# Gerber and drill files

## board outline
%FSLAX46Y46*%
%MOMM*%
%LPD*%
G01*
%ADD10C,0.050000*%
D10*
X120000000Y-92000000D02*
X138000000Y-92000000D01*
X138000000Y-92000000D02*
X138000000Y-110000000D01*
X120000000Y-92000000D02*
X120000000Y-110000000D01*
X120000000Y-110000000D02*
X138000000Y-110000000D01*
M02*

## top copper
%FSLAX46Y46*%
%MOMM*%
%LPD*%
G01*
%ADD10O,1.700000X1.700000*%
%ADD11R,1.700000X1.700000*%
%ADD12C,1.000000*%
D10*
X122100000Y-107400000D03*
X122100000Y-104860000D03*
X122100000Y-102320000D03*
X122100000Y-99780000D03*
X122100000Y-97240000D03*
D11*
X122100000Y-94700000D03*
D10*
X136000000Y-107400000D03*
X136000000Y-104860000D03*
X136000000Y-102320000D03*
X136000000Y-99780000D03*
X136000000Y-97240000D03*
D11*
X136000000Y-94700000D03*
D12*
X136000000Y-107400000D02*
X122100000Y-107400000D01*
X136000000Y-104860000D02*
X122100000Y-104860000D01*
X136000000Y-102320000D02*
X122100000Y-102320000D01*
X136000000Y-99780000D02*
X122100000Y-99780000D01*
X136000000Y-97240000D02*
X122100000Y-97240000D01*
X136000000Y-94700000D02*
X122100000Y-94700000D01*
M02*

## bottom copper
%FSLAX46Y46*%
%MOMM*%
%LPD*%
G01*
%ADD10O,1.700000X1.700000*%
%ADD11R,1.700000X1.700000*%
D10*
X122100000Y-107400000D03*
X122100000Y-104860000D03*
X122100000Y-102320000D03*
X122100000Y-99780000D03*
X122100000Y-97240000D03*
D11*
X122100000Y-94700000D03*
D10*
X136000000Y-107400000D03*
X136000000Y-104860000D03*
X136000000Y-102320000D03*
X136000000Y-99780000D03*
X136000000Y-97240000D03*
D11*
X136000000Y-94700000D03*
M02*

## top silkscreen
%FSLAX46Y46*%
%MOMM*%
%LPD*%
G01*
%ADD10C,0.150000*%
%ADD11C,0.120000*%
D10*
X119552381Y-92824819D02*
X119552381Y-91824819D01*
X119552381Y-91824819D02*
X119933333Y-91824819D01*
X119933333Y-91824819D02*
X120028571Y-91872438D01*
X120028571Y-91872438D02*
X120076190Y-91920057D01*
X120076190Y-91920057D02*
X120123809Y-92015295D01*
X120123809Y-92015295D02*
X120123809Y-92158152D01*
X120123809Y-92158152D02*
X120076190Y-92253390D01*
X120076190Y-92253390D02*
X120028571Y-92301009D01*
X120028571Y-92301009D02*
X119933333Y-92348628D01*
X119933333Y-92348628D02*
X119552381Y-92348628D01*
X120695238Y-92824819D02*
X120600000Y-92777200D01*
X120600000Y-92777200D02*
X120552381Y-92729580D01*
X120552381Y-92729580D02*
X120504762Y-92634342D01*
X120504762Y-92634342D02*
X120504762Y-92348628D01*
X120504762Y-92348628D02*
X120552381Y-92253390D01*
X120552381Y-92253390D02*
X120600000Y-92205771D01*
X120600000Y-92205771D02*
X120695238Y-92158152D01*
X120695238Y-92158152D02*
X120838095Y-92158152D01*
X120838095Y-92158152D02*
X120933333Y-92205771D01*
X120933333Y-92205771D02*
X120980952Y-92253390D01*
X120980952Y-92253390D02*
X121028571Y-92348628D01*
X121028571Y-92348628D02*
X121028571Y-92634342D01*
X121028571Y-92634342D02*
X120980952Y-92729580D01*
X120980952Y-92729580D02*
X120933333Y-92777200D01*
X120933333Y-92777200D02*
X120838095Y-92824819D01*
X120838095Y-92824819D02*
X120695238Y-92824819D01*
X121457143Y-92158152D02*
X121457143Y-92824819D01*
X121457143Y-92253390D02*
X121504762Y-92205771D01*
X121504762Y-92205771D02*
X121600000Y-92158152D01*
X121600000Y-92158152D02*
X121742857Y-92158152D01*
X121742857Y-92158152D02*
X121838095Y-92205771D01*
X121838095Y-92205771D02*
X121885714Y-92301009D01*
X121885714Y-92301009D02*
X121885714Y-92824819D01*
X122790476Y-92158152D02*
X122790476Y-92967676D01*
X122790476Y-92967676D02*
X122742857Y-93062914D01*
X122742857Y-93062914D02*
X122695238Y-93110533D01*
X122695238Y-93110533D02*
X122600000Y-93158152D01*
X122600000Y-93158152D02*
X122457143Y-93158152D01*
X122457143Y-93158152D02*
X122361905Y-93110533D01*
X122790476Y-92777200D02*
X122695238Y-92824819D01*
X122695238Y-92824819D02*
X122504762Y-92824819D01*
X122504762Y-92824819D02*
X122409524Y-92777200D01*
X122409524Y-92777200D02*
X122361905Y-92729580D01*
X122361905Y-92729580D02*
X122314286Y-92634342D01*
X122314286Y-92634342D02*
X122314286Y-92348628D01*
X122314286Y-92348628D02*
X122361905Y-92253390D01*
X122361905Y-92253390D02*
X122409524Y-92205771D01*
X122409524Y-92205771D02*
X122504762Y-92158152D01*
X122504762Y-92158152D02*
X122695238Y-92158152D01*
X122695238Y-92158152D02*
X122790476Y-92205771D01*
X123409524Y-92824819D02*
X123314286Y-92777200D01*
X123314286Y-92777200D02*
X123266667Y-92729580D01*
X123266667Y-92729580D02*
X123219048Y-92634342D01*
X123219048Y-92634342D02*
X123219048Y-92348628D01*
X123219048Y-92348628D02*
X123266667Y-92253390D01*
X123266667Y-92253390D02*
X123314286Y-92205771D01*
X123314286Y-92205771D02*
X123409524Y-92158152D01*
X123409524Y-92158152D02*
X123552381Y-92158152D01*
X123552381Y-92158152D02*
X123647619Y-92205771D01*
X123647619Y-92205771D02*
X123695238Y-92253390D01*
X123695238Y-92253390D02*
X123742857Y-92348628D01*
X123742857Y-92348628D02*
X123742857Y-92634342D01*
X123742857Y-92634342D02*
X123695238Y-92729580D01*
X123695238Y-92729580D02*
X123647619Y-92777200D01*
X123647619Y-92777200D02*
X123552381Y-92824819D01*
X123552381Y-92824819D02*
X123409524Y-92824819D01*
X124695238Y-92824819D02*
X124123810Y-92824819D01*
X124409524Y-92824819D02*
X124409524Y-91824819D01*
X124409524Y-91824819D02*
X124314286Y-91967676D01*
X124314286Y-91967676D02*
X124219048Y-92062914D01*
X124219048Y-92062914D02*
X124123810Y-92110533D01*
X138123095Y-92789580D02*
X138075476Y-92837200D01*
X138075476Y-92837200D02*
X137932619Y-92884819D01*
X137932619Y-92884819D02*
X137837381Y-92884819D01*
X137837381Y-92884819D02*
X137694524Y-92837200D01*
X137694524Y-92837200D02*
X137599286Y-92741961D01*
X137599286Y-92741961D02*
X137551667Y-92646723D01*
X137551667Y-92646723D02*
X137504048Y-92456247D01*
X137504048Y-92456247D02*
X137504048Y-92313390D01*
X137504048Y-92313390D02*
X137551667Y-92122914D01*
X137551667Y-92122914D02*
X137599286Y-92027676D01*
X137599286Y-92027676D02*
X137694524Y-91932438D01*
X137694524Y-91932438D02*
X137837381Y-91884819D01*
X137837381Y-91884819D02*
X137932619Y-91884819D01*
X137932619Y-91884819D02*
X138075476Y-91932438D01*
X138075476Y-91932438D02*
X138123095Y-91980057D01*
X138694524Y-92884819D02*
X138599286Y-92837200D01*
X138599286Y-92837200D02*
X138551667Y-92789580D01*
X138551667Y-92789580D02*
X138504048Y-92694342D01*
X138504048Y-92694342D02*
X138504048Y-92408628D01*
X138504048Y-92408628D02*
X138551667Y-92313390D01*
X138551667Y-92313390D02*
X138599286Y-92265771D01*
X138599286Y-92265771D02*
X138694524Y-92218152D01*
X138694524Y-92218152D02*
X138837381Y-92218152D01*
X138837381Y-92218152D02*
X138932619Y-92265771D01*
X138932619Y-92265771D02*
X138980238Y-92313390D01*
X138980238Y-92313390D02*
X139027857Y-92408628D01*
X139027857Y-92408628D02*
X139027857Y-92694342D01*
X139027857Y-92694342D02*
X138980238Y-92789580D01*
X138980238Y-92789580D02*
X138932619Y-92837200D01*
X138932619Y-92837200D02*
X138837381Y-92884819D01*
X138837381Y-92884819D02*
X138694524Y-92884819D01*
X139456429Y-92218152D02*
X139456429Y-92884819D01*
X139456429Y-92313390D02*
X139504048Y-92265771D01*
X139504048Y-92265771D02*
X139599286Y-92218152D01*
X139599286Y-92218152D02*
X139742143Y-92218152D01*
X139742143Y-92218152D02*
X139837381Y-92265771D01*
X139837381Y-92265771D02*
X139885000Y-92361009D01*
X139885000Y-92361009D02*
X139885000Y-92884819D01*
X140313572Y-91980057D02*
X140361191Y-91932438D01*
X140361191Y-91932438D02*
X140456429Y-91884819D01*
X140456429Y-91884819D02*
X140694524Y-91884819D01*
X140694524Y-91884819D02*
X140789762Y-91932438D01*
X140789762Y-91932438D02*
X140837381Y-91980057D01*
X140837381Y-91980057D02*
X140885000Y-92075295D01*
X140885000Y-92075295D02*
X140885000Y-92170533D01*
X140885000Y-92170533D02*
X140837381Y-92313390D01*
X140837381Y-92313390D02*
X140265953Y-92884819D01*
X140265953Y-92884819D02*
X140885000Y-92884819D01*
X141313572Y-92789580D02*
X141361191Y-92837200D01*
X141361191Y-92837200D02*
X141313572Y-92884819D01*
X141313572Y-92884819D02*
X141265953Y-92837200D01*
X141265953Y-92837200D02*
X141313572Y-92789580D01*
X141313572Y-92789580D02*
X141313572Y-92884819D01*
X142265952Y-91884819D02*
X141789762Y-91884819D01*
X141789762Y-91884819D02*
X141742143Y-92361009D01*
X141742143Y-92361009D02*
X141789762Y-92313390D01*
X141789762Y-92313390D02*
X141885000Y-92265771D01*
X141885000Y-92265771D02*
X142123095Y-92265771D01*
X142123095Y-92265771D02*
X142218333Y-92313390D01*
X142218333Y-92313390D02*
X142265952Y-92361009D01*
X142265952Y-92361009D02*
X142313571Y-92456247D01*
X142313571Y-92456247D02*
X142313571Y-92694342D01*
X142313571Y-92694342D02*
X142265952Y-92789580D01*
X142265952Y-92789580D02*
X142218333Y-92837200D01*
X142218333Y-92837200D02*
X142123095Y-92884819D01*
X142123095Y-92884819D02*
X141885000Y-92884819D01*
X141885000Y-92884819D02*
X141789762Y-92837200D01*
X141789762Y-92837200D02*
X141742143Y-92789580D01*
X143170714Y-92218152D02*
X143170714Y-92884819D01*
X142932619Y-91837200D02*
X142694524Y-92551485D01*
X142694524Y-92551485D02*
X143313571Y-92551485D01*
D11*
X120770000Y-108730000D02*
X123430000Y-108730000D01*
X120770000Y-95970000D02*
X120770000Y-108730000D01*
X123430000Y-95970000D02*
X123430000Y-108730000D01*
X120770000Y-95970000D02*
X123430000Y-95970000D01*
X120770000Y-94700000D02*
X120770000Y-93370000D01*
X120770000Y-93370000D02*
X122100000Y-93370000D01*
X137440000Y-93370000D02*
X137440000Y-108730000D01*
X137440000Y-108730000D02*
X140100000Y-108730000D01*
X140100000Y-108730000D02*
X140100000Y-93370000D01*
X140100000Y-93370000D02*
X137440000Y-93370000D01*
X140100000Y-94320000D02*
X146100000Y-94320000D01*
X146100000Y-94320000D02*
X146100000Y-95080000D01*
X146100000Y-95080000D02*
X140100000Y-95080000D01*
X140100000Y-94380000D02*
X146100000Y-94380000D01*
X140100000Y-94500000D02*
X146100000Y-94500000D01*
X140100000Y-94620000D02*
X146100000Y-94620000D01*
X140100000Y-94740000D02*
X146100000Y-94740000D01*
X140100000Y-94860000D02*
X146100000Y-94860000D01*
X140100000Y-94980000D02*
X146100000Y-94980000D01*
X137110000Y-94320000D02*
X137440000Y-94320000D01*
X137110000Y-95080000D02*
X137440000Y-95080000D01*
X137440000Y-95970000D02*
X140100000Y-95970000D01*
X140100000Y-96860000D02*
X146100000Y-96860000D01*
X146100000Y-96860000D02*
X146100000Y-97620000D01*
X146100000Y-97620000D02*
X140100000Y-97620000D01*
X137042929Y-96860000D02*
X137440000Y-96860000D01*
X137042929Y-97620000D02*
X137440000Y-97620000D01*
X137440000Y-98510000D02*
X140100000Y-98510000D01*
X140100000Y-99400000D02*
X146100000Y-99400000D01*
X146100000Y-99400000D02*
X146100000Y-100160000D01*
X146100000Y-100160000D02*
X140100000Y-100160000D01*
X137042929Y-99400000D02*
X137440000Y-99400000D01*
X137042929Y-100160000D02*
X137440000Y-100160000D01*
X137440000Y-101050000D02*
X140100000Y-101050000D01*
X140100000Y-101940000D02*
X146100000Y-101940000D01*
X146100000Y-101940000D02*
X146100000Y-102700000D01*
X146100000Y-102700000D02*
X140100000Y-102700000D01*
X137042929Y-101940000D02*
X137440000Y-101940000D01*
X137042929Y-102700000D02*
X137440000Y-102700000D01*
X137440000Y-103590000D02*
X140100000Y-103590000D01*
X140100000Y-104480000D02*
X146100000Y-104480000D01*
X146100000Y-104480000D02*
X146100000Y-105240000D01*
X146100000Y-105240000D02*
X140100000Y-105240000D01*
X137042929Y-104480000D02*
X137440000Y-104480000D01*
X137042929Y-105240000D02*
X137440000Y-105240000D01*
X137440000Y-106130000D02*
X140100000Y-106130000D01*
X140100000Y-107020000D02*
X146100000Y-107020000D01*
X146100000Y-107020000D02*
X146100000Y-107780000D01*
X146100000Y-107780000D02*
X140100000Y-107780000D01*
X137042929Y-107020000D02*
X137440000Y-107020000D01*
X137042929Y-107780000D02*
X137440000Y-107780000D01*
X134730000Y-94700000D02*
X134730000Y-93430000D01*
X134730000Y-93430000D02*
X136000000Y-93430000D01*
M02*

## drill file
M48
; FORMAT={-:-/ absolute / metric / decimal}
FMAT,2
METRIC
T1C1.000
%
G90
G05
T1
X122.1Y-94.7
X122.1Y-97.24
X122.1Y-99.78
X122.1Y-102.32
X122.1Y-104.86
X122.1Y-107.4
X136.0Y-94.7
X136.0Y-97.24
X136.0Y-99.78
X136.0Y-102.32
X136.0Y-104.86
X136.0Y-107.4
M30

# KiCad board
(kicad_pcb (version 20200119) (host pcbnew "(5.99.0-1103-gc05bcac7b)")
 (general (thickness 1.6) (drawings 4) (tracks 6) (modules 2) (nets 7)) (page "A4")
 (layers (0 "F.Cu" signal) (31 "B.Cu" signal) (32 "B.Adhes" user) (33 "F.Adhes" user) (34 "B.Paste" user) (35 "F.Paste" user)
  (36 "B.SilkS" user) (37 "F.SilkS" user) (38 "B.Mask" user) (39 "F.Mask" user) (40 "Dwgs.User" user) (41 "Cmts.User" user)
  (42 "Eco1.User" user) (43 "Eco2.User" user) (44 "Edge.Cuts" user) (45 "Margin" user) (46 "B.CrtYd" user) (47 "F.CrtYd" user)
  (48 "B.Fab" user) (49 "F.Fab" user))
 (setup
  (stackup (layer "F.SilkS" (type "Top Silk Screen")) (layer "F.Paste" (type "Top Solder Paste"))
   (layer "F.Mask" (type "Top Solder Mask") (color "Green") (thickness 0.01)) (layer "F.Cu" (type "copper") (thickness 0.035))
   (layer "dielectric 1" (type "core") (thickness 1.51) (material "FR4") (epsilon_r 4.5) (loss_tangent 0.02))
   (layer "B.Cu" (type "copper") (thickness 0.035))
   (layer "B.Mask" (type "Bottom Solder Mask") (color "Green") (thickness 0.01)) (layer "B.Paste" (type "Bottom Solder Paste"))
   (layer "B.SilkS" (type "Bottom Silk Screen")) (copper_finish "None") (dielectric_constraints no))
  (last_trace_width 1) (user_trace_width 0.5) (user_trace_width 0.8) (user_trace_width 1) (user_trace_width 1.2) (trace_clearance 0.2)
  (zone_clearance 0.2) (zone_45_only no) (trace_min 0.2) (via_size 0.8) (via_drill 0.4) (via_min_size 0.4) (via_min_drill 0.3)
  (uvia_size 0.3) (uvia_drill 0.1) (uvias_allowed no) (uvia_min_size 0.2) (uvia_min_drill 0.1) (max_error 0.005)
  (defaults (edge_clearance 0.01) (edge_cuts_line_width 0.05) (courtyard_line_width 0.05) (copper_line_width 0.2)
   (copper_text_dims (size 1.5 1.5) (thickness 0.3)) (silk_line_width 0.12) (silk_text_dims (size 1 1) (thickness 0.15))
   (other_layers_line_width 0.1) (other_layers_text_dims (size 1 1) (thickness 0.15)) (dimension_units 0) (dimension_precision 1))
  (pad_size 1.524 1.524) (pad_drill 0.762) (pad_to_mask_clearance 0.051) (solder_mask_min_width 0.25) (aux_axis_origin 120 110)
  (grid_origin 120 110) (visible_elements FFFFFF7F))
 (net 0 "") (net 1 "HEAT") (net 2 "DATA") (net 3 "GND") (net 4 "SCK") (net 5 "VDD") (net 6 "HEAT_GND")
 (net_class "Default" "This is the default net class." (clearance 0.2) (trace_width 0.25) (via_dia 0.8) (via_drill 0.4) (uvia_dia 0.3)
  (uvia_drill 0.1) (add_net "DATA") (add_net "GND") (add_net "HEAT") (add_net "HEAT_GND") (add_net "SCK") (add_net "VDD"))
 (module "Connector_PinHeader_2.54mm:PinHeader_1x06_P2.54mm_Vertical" (layer "F.Cu") (at 122.1 94.7)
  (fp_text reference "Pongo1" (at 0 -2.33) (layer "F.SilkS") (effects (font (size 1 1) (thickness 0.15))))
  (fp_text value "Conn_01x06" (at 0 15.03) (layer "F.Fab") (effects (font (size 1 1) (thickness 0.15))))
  (fp_line (start -1.33 14.03) (end 1.33 14.03) (layer "F.SilkS") (width 0.12))
  (fp_line (start -1.33 1.27) (end -1.33 14.03) (layer "F.SilkS") (width 0.12))
  (fp_line (start 1.33 1.27) (end 1.33 14.03) (layer "F.SilkS") (width 0.12))
  (fp_line (start -1.33 1.27) (end 1.33 1.27) (layer "F.SilkS") (width 0.12))
  (fp_line (start -1.33 0) (end -1.33 -1.33) (layer "F.SilkS") (width 0.12))
  (fp_line (start -1.33 -1.33) (end 0 -1.33) (layer "F.SilkS") (width 0.12))
  (pad "6" thru_hole oval (at 0 12.7) (size 1.7 1.7) (drill 1) (layers *.Cu *.Mask) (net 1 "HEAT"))
  (pad "5" thru_hole oval (at 0 10.16) (size 1.7 1.7) (drill 1) (layers *.Cu *.Mask) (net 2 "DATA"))
  (pad "4" thru_hole oval (at 0 7.62) (size 1.7 1.7) (drill 1) (layers *.Cu *.Mask) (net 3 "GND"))
  (pad "3" thru_hole oval (at 0 5.08) (size 1.7 1.7) (drill 1) (layers *.Cu *.Mask) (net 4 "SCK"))
  (pad "2" thru_hole oval (at 0 2.54) (size 1.7 1.7) (drill 1) (layers *.Cu *.Mask) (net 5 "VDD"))
  (pad "1" thru_hole rect (at 0 0) (size 1.7 1.7) (drill 1) (layers *.Cu *.Mask) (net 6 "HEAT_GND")))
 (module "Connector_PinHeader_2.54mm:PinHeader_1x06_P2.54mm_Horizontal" (layer "F.Cu") (at 136 94.7)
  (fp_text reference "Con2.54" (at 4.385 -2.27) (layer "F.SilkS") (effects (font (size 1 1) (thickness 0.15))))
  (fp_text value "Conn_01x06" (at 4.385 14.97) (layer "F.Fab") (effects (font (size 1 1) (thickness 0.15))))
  (fp_line (start 1.44 -1.33) (end 1.44 14.03) (layer "F.SilkS") (width 0.12))
  (fp_line (start 1.44 14.03) (end 4.1 14.03) (layer "F.SilkS") (width 0.12))
  (fp_line (start 4.1 14.03) (end 4.1 -1.33) (layer "F.SilkS") (width 0.12))
  (fp_line (start 4.1 -1.33) (end 1.44 -1.33) (layer "F.SilkS") (width 0.12))
  (fp_line (start 4.1 -0.38) (end 10.1 -0.38) (layer "F.SilkS") (width 0.12))
  (fp_line (start 10.1 -0.38) (end 10.1 0.38) (layer "F.SilkS") (width 0.12))
  (fp_line (start 10.1 0.38) (end 4.1 0.38) (layer "F.SilkS") (width 0.12))
  (fp_line (start 4.1 -0.32) (end 10.1 -0.32) (layer "F.SilkS") (width 0.12))
  (fp_line (start 4.1 -0.2) (end 10.1 -0.2) (layer "F.SilkS") (width 0.12))
  (fp_line (start 4.1 -0.08) (end 10.1 -0.08) (layer "F.SilkS") (width 0.12))
  (fp_line (start 4.1 0.04) (end 10.1 0.04) (layer "F.SilkS") (width 0.12))
  (fp_line (start 4.1 0.16) (end 10.1 0.16) (layer "F.SilkS") (width 0.12))
  (fp_line (start 4.1 0.28) (end 10.1 0.28) (layer "F.SilkS") (width 0.12))
  (fp_line (start 1.11 -0.38) (end 1.44 -0.38) (layer "F.SilkS") (width 0.12))
  (fp_line (start 1.11 0.38) (end 1.44 0.38) (layer "F.SilkS") (width 0.12))
  (fp_line (start 1.44 1.27) (end 4.1 1.27) (layer "F.SilkS") (width 0.12))
  (fp_line (start 4.1 2.16) (end 10.1 2.16) (layer "F.SilkS") (width 0.12))
  (fp_line (start 10.1 2.16) (end 10.1 2.92) (layer "F.SilkS") (width 0.12))
  (fp_line (start 10.1 2.92) (end 4.1 2.92) (layer "F.SilkS") (width 0.12))
  (fp_line (start 1.042929 2.16) (end 1.44 2.16) (layer "F.SilkS") (width 0.12))
  (fp_line (start 1.042929 2.92) (end 1.44 2.92) (layer "F.SilkS") (width 0.12))
  (fp_line (start 1.44 3.81) (end 4.1 3.81) (layer "F.SilkS") (width 0.12))
  (fp_line (start 4.1 4.7) (end 10.1 4.7) (layer "F.SilkS") (width 0.12))
  (fp_line (start 10.1 4.7) (end 10.1 5.46) (layer "F.SilkS") (width 0.12))
  (fp_line (start 10.1 5.46) (end 4.1 5.46) (layer "F.SilkS") (width 0.12))
  (fp_line (start 1.042929 4.7) (end 1.44 4.7) (layer "F.SilkS") (width 0.12))
  (fp_line (start 1.042929 5.46) (end 1.44 5.46) (layer "F.SilkS") (width 0.12))
  (fp_line (start 1.44 6.35) (end 4.1 6.35) (layer "F.SilkS") (width 0.12))
  (fp_line (start 4.1 7.24) (end 10.1 7.24) (layer "F.SilkS") (width 0.12))
  (fp_line (start 10.1 7.24) (end 10.1 8) (layer "F.SilkS") (width 0.12))
  (fp_line (start 10.1 8) (end 4.1 8) (layer "F.SilkS") (width 0.12))
  (fp_line (start 1.042929 7.24) (end 1.44 7.24) (layer "F.SilkS") (width 0.12))
  (fp_line (start 1.042929 8) (end 1.44 8) (layer "F.SilkS") (width 0.12))
  (fp_line (start 1.44 8.89) (end 4.1 8.89) (layer "F.SilkS") (width 0.12))
  (fp_line (start 4.1 9.78) (end 10.1 9.78) (layer "F.SilkS") (width 0.12))
  (fp_line (start 10.1 9.78) (end 10.1 10.54) (layer "F.SilkS") (width 0.12))
  (fp_line (start 10.1 10.54) (end 4.1 10.54) (layer "F.SilkS") (width 0.12))
  (fp_line (start 1.042929 9.78) (end 1.44 9.78) (layer "F.SilkS") (width 0.12))
  (fp_line (start 1.042929 10.54) (end 1.44 10.54) (layer "F.SilkS") (width 0.12))
  (fp_line (start 1.44 11.43) (end 4.1 11.43) (layer "F.SilkS") (width 0.12))
  (fp_line (start 4.1 12.32) (end 10.1 12.32) (layer "F.SilkS") (width 0.12))
  (fp_line (start 10.1 12.32) (end 10.1 13.08) (layer "F.SilkS") (width 0.12))
  (fp_line (start 10.1 13.08) (end 4.1 13.08) (layer "F.SilkS") (width 0.12))
  (fp_line (start 1.042929 12.32) (end 1.44 12.32) (layer "F.SilkS") (width 0.12))
  (fp_line (start 1.042929 13.08) (end 1.44 13.08) (layer "F.SilkS") (width 0.12))
  (fp_line (start -1.27 0) (end -1.27 -1.27) (layer "F.SilkS") (width 0.12))
  (fp_line (start -1.27 -1.27) (end 0 -1.27) (layer "F.SilkS") (width 0.12))
  (pad "6" thru_hole oval (at 0 12.7) (size 1.7 1.7) (drill 1) (layers *.Cu *.Mask) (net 1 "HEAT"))
  (pad "5" thru_hole oval (at 0 10.16) (size 1.7 1.7) (drill 1) (layers *.Cu *.Mask) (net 2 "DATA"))
  (pad "4" thru_hole oval (at 0 7.62) (size 1.7 1.7) (drill 1) (layers *.Cu *.Mask) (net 3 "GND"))
  (pad "3" thru_hole oval (at 0 5.08) (size 1.7 1.7) (drill 1) (layers *.Cu *.Mask) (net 4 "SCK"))
  (pad "2" thru_hole oval (at 0 2.54) (size 1.7 1.7) (drill 1) (layers *.Cu *.Mask) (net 5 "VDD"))
  (pad "1" thru_hole rect (at 0 0) (size 1.7 1.7) (drill 1) (layers *.Cu *.Mask) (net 6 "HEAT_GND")))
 (gr_line (start 120 92) (end 138 92) (layer "Edge.Cuts") (width 0.05))
 (gr_line (start 138 92) (end 138 110) (layer "Edge.Cuts") (width 0.05))
 (gr_line (start 120 92) (end 120 110) (layer "Edge.Cuts") (width 0.05))
 (gr_line (start 120 110) (end 138 110) (layer "Edge.Cuts") (width 0.05))
 (segment (start 136 107.4) (end 122.1 107.4) (width 1) (layer "F.Cu") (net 1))
 (segment (start 136 104.86) (end 122.1 104.86) (width 1) (layer "F.Cu") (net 2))
 (segment (start 136 102.32) (end 122.1 102.32) (width 1) (layer "F.Cu") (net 3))
 (segment (start 136 99.78) (end 122.1 99.78) (width 1) (layer "F.Cu") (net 4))
 (segment (start 136 97.24) (end 122.1 97.24) (width 1) (layer "F.Cu") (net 5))
 (segment (start 136 94.7) (end 122.1 94.7) (width 1) (layer "F.Cu") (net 6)))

